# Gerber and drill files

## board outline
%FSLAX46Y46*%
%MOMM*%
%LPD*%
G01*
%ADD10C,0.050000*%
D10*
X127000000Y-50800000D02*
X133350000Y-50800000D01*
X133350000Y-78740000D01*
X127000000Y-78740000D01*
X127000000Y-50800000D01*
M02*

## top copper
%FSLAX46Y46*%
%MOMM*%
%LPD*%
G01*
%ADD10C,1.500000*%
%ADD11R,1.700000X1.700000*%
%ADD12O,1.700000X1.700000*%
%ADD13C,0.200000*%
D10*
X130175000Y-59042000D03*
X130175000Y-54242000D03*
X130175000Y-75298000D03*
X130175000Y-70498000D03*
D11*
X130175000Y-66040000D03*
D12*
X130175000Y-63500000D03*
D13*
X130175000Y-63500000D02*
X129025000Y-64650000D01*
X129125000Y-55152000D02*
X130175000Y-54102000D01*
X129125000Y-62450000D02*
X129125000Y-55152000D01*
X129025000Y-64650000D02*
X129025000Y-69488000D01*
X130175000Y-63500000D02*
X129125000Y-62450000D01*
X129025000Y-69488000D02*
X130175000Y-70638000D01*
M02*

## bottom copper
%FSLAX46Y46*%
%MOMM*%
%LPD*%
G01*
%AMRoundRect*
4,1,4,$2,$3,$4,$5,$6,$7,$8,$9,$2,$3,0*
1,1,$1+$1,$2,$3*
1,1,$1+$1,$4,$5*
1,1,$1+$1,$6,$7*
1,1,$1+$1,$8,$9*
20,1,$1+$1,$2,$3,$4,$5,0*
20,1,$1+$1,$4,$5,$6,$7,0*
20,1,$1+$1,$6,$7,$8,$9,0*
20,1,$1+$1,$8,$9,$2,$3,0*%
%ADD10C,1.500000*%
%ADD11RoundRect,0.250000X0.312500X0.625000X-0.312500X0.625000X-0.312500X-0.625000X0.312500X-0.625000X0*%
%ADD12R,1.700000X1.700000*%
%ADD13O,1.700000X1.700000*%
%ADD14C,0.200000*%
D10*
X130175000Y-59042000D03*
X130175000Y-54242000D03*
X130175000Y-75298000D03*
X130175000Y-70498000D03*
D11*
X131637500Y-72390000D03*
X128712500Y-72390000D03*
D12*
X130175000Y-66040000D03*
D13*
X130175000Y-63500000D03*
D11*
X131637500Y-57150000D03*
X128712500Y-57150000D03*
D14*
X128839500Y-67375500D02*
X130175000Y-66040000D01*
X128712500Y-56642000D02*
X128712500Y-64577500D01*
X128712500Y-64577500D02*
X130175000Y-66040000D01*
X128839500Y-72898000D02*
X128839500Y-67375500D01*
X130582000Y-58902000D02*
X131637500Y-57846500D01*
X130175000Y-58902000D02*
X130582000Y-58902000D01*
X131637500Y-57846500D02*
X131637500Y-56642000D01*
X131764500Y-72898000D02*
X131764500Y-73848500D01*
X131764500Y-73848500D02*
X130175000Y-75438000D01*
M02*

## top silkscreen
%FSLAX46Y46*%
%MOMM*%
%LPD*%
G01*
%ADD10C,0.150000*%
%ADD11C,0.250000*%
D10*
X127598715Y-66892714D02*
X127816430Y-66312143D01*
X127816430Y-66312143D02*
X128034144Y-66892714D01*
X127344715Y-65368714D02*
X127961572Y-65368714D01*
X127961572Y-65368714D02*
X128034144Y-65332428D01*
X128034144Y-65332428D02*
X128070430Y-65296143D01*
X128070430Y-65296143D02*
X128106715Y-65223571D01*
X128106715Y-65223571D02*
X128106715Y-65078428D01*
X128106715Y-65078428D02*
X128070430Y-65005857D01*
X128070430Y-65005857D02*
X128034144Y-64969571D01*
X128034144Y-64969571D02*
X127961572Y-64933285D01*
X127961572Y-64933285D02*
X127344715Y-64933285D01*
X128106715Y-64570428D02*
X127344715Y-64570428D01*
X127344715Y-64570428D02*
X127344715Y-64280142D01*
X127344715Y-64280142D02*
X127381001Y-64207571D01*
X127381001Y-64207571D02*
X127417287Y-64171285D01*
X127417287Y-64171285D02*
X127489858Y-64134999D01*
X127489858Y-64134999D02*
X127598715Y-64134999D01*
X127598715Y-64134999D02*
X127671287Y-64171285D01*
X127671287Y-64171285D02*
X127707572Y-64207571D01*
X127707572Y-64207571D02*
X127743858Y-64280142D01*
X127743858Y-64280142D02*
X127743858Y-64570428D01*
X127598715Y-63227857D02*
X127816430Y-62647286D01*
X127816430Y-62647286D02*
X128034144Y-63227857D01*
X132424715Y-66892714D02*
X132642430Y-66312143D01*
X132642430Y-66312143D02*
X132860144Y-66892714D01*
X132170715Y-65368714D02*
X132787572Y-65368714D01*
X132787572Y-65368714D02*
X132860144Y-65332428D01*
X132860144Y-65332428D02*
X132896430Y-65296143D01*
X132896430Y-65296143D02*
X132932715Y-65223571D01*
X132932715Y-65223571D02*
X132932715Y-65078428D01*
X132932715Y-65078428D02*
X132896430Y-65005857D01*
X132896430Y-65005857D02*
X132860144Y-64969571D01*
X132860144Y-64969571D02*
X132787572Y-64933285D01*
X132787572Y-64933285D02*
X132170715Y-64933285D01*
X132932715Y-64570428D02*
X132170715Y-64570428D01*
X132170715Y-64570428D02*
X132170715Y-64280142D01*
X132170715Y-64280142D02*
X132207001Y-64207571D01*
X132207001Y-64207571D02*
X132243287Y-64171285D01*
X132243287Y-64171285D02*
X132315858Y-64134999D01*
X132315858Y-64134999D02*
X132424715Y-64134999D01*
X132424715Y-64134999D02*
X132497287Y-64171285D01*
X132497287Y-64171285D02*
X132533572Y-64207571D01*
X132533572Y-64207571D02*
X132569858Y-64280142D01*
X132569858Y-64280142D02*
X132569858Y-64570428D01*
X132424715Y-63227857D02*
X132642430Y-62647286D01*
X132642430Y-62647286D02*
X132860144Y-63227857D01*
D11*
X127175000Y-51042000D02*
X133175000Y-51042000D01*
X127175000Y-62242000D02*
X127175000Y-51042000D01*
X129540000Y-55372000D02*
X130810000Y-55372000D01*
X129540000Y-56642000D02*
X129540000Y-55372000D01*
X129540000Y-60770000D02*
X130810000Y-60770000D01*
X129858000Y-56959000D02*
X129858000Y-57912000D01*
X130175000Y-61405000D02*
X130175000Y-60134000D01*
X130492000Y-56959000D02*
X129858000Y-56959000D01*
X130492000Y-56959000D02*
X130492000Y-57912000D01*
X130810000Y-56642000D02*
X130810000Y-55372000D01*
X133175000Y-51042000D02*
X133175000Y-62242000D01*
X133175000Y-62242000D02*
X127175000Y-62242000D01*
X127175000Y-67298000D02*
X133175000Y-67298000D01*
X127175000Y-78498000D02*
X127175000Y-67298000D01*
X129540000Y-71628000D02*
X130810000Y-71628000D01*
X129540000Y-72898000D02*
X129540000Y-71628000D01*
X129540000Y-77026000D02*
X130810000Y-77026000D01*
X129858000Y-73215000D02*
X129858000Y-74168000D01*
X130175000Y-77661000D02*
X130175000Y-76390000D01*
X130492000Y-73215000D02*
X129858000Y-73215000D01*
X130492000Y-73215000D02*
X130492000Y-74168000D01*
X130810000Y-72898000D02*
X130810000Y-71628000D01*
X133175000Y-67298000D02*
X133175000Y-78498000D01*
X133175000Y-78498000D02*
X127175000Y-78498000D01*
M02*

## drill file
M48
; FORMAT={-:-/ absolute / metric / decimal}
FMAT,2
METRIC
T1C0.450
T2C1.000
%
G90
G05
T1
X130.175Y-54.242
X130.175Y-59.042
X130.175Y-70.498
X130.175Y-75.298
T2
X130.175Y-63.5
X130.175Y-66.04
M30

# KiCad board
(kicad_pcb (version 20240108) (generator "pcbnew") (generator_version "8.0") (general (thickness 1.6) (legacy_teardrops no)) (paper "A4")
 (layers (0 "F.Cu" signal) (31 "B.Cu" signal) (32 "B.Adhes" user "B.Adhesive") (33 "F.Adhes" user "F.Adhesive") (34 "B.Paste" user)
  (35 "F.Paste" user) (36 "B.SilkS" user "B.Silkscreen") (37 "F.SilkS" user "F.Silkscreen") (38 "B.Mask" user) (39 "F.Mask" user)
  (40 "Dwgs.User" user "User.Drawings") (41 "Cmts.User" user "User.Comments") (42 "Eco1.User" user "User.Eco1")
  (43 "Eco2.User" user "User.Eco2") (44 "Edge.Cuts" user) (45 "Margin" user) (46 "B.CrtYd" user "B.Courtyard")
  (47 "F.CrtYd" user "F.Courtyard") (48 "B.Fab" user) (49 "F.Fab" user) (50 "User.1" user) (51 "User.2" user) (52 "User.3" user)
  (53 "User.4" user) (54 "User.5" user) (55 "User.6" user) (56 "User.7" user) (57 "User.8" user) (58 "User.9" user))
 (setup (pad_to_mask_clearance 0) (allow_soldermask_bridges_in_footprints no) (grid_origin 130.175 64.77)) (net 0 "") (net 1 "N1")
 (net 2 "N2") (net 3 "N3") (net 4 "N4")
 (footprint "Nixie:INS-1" (layer "F.Cu") (at 130.175 56.642 90)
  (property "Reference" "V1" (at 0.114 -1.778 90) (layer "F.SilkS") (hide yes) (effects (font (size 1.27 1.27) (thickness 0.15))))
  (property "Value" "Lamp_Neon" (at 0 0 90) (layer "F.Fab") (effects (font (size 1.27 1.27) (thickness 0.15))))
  (fp_line (start 5.6 -3) (end 5.6 3) (stroke (width 0.25) (type solid)) (layer "F.SilkS"))
  (fp_line (start -5.6 -3) (end 5.6 -3) (stroke (width 0.25) (type solid)) (layer "F.SilkS"))
  (fp_line (start 1.27 -0.635) (end 1.27 0.635) (stroke (width 0.25) (type solid)) (layer "F.SilkS"))
  (fp_line (start 0 -0.635) (end 1.27 -0.635) (stroke (width 0.25) (type solid)) (layer "F.SilkS"))
  (fp_line (start -4.128 -0.635) (end -4.128 0.635) (stroke (width 0.25) (type solid)) (layer "F.SilkS"))
  (fp_line (start -0.317 -0.317) (end -1.27 -0.317) (stroke (width 0.25) (type solid)) (layer "F.SilkS"))
  (fp_line (start -4.763 0) (end -3.492 0) (stroke (width 0.25) (type solid)) (layer "F.SilkS"))
  (fp_line (start -0.317 0.317) (end -0.317 -0.317) (stroke (width 0.25) (type solid)) (layer "F.SilkS"))
  (fp_line (start -0.317 0.317) (end -1.27 0.317) (stroke (width 0.25) (type solid)) (layer "F.SilkS"))
  (fp_line (start 0 0.635) (end 1.27 0.635) (stroke (width 0.25) (type solid)) (layer "F.SilkS"))
  (fp_line (start 5.6 3) (end -5.6 3) (stroke (width 0.25) (type solid)) (layer "F.SilkS"))
  (fp_line (start -5.6 3) (end -5.6 -3) (stroke (width 0.25) (type solid)) (layer "F.SilkS"))
  (pad "1" thru_hole circle (at -2.4 0 90) (size 1.5 1.5) (drill 0.45) (layers "*.Cu" "*.Mask") (remove_unused_layers no) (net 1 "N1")
   (solder_mask_margin 0.1016) (zone_connect 2) (thermal_bridge_angle 0))
  (pad "2" thru_hole circle (at 2.4 0 90) (size 1.5 1.5) (drill 0.45) (layers "*.Cu" "*.Mask") (remove_unused_layers no) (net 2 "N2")
   (solder_mask_margin 0.1016) (zone_connect 2) (thermal_bridge_angle 0)))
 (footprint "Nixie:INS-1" (layer "F.Cu") (at 130.175 72.898 90)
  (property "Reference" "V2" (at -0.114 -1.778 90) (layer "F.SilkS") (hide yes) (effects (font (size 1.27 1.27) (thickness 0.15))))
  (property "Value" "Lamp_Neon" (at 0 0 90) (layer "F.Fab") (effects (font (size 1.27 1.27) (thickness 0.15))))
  (fp_line (start 5.6 -3) (end 5.6 3) (stroke (width 0.25) (type solid)) (layer "F.SilkS"))
  (fp_line (start -5.6 -3) (end 5.6 -3) (stroke (width 0.25) (type solid)) (layer "F.SilkS"))
  (fp_line (start 1.27 -0.635) (end 1.27 0.635) (stroke (width 0.25) (type solid)) (layer "F.SilkS"))
  (fp_line (start 0 -0.635) (end 1.27 -0.635) (stroke (width 0.25) (type solid)) (layer "F.SilkS"))
  (fp_line (start -4.128 -0.635) (end -4.128 0.635) (stroke (width 0.25) (type solid)) (layer "F.SilkS"))
  (fp_line (start -0.317 -0.317) (end -1.27 -0.317) (stroke (width 0.25) (type solid)) (layer "F.SilkS"))
  (fp_line (start -4.763 0) (end -3.492 0) (stroke (width 0.25) (type solid)) (layer "F.SilkS"))
  (fp_line (start -0.317 0.317) (end -0.317 -0.317) (stroke (width 0.25) (type solid)) (layer "F.SilkS"))
  (fp_line (start -0.317 0.317) (end -1.27 0.317) (stroke (width 0.25) (type solid)) (layer "F.SilkS"))
  (fp_line (start 0 0.635) (end 1.27 0.635) (stroke (width 0.25) (type solid)) (layer "F.SilkS"))
  (fp_line (start 5.6 3) (end -5.6 3) (stroke (width 0.25) (type solid)) (layer "F.SilkS"))
  (fp_line (start -5.6 3) (end -5.6 -3) (stroke (width 0.25) (type solid)) (layer "F.SilkS"))
  (pad "1" thru_hole circle (at -2.4 0 90) (size 1.5 1.5) (drill 0.45) (layers "*.Cu" "*.Mask") (remove_unused_layers no) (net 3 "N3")
   (solder_mask_margin 0.1016) (zone_connect 2) (thermal_bridge_angle 0))
  (pad "2" thru_hole circle (at 2.4 0 90) (size 1.5 1.5) (drill 0.45) (layers "*.Cu" "*.Mask") (remove_unused_layers no) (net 2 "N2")
   (solder_mask_margin 0.1016) (zone_connect 2) (thermal_bridge_angle 0)))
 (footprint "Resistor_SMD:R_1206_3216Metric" (layer "B.Cu") (at 130.175 72.39 180)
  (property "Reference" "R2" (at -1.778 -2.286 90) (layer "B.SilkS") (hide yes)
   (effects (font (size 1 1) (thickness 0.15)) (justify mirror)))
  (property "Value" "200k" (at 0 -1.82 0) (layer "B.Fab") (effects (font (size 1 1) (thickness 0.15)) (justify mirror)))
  (pad "1" smd roundrect (at -1.4625 0 180) (size 1.125 1.75) (layers "B.Cu" "B.Paste" "B.Mask") (roundrect_rratio 0.222222) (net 3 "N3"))
  (pad "2" smd roundrect (at 1.4625 0 180) (size 1.125 1.75) (layers "B.Cu" "B.Paste" "B.Mask") (roundrect_rratio 0.222222) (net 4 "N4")))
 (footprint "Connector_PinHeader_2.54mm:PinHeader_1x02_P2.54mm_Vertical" (layer "B.Cu") (at 130.175 66.04)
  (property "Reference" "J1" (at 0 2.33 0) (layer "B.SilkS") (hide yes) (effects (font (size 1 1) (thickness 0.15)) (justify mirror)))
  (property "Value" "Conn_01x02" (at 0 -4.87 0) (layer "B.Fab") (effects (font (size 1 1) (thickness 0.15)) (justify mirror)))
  (pad "1" thru_hole rect (at 0 0) (size 1.7 1.7) (drill 1) (layers "*.Cu" "*.Mask") (remove_unused_layers no) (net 4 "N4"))
  (pad "2" thru_hole oval (at 0 -2.54) (size 1.7 1.7) (drill 1) (layers "*.Cu" "*.Mask") (remove_unused_layers no) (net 2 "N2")))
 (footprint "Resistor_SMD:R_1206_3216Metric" (layer "B.Cu") (at 130.175 57.15 180)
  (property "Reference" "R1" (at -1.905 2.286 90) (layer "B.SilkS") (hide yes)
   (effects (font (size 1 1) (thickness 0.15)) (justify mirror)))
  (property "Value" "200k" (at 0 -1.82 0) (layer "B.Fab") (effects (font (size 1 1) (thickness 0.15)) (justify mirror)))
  (pad "1" smd roundrect (at -1.4625 0 180) (size 1.125 1.75) (layers "B.Cu" "B.Paste" "B.Mask") (roundrect_rratio 0.222222) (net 1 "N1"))
  (pad "2" smd roundrect (at 1.4625 0 180) (size 1.125 1.75) (layers "B.Cu" "B.Paste" "B.Mask") (roundrect_rratio 0.222222) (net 4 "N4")))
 (gr_rect (start 127 50.8) (end 133.35 78.74) (stroke (width 0.05) (type default)) (fill none) (layer "Edge.Cuts"))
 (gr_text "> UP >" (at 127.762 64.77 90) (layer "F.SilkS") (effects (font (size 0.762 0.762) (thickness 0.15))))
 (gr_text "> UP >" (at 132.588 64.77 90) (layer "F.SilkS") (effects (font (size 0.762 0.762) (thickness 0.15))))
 (segment (start 130.175 63.5) (end 129.025 64.65) (width 0.2) (layer "F.Cu") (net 2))
 (segment (start 129.125 55.152) (end 130.175 54.102) (width 0.2) (layer "F.Cu") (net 2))
 (segment (start 129.125 62.45) (end 129.125 55.152) (width 0.2) (layer "F.Cu") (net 2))
 (segment (start 129.025 64.65) (end 129.025 69.488) (width 0.2) (layer "F.Cu") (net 2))
 (segment (start 130.175 63.5) (end 129.125 62.45) (width 0.2) (layer "F.Cu") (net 2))
 (segment (start 129.025 69.488) (end 130.175 70.638) (width 0.2) (layer "F.Cu") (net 2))
 (segment (start 128.8395 67.3755) (end 130.175 66.04) (width 0.2) (layer "B.Cu") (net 4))
 (segment (start 128.7125 56.642) (end 128.7125 64.5775) (width 0.2) (layer "B.Cu") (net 4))
 (segment (start 128.7125 64.5775) (end 130.175 66.04) (width 0.2) (layer "B.Cu") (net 4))
 (segment (start 128.8395 72.898) (end 128.8395 67.3755) (width 0.2) (layer "B.Cu") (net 4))
 (segment (start 130.582 58.902) (end 131.6375 57.8465) (width 0.2) (layer "B.Cu") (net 1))
 (segment (start 130.175 58.902) (end 130.582 58.902) (width 0.2) (layer "B.Cu") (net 1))
 (segment (start 131.6375 57.8465) (end 131.6375 56.642) (width 0.2) (layer "B.Cu") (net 1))
 (segment (start 131.7645 72.898) (end 131.7645 73.8485) (width 0.2) (layer "B.Cu") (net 3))
 (segment (start 131.7645 73.8485) (end 130.175 75.438) (width 0.2) (layer "B.Cu") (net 3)))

